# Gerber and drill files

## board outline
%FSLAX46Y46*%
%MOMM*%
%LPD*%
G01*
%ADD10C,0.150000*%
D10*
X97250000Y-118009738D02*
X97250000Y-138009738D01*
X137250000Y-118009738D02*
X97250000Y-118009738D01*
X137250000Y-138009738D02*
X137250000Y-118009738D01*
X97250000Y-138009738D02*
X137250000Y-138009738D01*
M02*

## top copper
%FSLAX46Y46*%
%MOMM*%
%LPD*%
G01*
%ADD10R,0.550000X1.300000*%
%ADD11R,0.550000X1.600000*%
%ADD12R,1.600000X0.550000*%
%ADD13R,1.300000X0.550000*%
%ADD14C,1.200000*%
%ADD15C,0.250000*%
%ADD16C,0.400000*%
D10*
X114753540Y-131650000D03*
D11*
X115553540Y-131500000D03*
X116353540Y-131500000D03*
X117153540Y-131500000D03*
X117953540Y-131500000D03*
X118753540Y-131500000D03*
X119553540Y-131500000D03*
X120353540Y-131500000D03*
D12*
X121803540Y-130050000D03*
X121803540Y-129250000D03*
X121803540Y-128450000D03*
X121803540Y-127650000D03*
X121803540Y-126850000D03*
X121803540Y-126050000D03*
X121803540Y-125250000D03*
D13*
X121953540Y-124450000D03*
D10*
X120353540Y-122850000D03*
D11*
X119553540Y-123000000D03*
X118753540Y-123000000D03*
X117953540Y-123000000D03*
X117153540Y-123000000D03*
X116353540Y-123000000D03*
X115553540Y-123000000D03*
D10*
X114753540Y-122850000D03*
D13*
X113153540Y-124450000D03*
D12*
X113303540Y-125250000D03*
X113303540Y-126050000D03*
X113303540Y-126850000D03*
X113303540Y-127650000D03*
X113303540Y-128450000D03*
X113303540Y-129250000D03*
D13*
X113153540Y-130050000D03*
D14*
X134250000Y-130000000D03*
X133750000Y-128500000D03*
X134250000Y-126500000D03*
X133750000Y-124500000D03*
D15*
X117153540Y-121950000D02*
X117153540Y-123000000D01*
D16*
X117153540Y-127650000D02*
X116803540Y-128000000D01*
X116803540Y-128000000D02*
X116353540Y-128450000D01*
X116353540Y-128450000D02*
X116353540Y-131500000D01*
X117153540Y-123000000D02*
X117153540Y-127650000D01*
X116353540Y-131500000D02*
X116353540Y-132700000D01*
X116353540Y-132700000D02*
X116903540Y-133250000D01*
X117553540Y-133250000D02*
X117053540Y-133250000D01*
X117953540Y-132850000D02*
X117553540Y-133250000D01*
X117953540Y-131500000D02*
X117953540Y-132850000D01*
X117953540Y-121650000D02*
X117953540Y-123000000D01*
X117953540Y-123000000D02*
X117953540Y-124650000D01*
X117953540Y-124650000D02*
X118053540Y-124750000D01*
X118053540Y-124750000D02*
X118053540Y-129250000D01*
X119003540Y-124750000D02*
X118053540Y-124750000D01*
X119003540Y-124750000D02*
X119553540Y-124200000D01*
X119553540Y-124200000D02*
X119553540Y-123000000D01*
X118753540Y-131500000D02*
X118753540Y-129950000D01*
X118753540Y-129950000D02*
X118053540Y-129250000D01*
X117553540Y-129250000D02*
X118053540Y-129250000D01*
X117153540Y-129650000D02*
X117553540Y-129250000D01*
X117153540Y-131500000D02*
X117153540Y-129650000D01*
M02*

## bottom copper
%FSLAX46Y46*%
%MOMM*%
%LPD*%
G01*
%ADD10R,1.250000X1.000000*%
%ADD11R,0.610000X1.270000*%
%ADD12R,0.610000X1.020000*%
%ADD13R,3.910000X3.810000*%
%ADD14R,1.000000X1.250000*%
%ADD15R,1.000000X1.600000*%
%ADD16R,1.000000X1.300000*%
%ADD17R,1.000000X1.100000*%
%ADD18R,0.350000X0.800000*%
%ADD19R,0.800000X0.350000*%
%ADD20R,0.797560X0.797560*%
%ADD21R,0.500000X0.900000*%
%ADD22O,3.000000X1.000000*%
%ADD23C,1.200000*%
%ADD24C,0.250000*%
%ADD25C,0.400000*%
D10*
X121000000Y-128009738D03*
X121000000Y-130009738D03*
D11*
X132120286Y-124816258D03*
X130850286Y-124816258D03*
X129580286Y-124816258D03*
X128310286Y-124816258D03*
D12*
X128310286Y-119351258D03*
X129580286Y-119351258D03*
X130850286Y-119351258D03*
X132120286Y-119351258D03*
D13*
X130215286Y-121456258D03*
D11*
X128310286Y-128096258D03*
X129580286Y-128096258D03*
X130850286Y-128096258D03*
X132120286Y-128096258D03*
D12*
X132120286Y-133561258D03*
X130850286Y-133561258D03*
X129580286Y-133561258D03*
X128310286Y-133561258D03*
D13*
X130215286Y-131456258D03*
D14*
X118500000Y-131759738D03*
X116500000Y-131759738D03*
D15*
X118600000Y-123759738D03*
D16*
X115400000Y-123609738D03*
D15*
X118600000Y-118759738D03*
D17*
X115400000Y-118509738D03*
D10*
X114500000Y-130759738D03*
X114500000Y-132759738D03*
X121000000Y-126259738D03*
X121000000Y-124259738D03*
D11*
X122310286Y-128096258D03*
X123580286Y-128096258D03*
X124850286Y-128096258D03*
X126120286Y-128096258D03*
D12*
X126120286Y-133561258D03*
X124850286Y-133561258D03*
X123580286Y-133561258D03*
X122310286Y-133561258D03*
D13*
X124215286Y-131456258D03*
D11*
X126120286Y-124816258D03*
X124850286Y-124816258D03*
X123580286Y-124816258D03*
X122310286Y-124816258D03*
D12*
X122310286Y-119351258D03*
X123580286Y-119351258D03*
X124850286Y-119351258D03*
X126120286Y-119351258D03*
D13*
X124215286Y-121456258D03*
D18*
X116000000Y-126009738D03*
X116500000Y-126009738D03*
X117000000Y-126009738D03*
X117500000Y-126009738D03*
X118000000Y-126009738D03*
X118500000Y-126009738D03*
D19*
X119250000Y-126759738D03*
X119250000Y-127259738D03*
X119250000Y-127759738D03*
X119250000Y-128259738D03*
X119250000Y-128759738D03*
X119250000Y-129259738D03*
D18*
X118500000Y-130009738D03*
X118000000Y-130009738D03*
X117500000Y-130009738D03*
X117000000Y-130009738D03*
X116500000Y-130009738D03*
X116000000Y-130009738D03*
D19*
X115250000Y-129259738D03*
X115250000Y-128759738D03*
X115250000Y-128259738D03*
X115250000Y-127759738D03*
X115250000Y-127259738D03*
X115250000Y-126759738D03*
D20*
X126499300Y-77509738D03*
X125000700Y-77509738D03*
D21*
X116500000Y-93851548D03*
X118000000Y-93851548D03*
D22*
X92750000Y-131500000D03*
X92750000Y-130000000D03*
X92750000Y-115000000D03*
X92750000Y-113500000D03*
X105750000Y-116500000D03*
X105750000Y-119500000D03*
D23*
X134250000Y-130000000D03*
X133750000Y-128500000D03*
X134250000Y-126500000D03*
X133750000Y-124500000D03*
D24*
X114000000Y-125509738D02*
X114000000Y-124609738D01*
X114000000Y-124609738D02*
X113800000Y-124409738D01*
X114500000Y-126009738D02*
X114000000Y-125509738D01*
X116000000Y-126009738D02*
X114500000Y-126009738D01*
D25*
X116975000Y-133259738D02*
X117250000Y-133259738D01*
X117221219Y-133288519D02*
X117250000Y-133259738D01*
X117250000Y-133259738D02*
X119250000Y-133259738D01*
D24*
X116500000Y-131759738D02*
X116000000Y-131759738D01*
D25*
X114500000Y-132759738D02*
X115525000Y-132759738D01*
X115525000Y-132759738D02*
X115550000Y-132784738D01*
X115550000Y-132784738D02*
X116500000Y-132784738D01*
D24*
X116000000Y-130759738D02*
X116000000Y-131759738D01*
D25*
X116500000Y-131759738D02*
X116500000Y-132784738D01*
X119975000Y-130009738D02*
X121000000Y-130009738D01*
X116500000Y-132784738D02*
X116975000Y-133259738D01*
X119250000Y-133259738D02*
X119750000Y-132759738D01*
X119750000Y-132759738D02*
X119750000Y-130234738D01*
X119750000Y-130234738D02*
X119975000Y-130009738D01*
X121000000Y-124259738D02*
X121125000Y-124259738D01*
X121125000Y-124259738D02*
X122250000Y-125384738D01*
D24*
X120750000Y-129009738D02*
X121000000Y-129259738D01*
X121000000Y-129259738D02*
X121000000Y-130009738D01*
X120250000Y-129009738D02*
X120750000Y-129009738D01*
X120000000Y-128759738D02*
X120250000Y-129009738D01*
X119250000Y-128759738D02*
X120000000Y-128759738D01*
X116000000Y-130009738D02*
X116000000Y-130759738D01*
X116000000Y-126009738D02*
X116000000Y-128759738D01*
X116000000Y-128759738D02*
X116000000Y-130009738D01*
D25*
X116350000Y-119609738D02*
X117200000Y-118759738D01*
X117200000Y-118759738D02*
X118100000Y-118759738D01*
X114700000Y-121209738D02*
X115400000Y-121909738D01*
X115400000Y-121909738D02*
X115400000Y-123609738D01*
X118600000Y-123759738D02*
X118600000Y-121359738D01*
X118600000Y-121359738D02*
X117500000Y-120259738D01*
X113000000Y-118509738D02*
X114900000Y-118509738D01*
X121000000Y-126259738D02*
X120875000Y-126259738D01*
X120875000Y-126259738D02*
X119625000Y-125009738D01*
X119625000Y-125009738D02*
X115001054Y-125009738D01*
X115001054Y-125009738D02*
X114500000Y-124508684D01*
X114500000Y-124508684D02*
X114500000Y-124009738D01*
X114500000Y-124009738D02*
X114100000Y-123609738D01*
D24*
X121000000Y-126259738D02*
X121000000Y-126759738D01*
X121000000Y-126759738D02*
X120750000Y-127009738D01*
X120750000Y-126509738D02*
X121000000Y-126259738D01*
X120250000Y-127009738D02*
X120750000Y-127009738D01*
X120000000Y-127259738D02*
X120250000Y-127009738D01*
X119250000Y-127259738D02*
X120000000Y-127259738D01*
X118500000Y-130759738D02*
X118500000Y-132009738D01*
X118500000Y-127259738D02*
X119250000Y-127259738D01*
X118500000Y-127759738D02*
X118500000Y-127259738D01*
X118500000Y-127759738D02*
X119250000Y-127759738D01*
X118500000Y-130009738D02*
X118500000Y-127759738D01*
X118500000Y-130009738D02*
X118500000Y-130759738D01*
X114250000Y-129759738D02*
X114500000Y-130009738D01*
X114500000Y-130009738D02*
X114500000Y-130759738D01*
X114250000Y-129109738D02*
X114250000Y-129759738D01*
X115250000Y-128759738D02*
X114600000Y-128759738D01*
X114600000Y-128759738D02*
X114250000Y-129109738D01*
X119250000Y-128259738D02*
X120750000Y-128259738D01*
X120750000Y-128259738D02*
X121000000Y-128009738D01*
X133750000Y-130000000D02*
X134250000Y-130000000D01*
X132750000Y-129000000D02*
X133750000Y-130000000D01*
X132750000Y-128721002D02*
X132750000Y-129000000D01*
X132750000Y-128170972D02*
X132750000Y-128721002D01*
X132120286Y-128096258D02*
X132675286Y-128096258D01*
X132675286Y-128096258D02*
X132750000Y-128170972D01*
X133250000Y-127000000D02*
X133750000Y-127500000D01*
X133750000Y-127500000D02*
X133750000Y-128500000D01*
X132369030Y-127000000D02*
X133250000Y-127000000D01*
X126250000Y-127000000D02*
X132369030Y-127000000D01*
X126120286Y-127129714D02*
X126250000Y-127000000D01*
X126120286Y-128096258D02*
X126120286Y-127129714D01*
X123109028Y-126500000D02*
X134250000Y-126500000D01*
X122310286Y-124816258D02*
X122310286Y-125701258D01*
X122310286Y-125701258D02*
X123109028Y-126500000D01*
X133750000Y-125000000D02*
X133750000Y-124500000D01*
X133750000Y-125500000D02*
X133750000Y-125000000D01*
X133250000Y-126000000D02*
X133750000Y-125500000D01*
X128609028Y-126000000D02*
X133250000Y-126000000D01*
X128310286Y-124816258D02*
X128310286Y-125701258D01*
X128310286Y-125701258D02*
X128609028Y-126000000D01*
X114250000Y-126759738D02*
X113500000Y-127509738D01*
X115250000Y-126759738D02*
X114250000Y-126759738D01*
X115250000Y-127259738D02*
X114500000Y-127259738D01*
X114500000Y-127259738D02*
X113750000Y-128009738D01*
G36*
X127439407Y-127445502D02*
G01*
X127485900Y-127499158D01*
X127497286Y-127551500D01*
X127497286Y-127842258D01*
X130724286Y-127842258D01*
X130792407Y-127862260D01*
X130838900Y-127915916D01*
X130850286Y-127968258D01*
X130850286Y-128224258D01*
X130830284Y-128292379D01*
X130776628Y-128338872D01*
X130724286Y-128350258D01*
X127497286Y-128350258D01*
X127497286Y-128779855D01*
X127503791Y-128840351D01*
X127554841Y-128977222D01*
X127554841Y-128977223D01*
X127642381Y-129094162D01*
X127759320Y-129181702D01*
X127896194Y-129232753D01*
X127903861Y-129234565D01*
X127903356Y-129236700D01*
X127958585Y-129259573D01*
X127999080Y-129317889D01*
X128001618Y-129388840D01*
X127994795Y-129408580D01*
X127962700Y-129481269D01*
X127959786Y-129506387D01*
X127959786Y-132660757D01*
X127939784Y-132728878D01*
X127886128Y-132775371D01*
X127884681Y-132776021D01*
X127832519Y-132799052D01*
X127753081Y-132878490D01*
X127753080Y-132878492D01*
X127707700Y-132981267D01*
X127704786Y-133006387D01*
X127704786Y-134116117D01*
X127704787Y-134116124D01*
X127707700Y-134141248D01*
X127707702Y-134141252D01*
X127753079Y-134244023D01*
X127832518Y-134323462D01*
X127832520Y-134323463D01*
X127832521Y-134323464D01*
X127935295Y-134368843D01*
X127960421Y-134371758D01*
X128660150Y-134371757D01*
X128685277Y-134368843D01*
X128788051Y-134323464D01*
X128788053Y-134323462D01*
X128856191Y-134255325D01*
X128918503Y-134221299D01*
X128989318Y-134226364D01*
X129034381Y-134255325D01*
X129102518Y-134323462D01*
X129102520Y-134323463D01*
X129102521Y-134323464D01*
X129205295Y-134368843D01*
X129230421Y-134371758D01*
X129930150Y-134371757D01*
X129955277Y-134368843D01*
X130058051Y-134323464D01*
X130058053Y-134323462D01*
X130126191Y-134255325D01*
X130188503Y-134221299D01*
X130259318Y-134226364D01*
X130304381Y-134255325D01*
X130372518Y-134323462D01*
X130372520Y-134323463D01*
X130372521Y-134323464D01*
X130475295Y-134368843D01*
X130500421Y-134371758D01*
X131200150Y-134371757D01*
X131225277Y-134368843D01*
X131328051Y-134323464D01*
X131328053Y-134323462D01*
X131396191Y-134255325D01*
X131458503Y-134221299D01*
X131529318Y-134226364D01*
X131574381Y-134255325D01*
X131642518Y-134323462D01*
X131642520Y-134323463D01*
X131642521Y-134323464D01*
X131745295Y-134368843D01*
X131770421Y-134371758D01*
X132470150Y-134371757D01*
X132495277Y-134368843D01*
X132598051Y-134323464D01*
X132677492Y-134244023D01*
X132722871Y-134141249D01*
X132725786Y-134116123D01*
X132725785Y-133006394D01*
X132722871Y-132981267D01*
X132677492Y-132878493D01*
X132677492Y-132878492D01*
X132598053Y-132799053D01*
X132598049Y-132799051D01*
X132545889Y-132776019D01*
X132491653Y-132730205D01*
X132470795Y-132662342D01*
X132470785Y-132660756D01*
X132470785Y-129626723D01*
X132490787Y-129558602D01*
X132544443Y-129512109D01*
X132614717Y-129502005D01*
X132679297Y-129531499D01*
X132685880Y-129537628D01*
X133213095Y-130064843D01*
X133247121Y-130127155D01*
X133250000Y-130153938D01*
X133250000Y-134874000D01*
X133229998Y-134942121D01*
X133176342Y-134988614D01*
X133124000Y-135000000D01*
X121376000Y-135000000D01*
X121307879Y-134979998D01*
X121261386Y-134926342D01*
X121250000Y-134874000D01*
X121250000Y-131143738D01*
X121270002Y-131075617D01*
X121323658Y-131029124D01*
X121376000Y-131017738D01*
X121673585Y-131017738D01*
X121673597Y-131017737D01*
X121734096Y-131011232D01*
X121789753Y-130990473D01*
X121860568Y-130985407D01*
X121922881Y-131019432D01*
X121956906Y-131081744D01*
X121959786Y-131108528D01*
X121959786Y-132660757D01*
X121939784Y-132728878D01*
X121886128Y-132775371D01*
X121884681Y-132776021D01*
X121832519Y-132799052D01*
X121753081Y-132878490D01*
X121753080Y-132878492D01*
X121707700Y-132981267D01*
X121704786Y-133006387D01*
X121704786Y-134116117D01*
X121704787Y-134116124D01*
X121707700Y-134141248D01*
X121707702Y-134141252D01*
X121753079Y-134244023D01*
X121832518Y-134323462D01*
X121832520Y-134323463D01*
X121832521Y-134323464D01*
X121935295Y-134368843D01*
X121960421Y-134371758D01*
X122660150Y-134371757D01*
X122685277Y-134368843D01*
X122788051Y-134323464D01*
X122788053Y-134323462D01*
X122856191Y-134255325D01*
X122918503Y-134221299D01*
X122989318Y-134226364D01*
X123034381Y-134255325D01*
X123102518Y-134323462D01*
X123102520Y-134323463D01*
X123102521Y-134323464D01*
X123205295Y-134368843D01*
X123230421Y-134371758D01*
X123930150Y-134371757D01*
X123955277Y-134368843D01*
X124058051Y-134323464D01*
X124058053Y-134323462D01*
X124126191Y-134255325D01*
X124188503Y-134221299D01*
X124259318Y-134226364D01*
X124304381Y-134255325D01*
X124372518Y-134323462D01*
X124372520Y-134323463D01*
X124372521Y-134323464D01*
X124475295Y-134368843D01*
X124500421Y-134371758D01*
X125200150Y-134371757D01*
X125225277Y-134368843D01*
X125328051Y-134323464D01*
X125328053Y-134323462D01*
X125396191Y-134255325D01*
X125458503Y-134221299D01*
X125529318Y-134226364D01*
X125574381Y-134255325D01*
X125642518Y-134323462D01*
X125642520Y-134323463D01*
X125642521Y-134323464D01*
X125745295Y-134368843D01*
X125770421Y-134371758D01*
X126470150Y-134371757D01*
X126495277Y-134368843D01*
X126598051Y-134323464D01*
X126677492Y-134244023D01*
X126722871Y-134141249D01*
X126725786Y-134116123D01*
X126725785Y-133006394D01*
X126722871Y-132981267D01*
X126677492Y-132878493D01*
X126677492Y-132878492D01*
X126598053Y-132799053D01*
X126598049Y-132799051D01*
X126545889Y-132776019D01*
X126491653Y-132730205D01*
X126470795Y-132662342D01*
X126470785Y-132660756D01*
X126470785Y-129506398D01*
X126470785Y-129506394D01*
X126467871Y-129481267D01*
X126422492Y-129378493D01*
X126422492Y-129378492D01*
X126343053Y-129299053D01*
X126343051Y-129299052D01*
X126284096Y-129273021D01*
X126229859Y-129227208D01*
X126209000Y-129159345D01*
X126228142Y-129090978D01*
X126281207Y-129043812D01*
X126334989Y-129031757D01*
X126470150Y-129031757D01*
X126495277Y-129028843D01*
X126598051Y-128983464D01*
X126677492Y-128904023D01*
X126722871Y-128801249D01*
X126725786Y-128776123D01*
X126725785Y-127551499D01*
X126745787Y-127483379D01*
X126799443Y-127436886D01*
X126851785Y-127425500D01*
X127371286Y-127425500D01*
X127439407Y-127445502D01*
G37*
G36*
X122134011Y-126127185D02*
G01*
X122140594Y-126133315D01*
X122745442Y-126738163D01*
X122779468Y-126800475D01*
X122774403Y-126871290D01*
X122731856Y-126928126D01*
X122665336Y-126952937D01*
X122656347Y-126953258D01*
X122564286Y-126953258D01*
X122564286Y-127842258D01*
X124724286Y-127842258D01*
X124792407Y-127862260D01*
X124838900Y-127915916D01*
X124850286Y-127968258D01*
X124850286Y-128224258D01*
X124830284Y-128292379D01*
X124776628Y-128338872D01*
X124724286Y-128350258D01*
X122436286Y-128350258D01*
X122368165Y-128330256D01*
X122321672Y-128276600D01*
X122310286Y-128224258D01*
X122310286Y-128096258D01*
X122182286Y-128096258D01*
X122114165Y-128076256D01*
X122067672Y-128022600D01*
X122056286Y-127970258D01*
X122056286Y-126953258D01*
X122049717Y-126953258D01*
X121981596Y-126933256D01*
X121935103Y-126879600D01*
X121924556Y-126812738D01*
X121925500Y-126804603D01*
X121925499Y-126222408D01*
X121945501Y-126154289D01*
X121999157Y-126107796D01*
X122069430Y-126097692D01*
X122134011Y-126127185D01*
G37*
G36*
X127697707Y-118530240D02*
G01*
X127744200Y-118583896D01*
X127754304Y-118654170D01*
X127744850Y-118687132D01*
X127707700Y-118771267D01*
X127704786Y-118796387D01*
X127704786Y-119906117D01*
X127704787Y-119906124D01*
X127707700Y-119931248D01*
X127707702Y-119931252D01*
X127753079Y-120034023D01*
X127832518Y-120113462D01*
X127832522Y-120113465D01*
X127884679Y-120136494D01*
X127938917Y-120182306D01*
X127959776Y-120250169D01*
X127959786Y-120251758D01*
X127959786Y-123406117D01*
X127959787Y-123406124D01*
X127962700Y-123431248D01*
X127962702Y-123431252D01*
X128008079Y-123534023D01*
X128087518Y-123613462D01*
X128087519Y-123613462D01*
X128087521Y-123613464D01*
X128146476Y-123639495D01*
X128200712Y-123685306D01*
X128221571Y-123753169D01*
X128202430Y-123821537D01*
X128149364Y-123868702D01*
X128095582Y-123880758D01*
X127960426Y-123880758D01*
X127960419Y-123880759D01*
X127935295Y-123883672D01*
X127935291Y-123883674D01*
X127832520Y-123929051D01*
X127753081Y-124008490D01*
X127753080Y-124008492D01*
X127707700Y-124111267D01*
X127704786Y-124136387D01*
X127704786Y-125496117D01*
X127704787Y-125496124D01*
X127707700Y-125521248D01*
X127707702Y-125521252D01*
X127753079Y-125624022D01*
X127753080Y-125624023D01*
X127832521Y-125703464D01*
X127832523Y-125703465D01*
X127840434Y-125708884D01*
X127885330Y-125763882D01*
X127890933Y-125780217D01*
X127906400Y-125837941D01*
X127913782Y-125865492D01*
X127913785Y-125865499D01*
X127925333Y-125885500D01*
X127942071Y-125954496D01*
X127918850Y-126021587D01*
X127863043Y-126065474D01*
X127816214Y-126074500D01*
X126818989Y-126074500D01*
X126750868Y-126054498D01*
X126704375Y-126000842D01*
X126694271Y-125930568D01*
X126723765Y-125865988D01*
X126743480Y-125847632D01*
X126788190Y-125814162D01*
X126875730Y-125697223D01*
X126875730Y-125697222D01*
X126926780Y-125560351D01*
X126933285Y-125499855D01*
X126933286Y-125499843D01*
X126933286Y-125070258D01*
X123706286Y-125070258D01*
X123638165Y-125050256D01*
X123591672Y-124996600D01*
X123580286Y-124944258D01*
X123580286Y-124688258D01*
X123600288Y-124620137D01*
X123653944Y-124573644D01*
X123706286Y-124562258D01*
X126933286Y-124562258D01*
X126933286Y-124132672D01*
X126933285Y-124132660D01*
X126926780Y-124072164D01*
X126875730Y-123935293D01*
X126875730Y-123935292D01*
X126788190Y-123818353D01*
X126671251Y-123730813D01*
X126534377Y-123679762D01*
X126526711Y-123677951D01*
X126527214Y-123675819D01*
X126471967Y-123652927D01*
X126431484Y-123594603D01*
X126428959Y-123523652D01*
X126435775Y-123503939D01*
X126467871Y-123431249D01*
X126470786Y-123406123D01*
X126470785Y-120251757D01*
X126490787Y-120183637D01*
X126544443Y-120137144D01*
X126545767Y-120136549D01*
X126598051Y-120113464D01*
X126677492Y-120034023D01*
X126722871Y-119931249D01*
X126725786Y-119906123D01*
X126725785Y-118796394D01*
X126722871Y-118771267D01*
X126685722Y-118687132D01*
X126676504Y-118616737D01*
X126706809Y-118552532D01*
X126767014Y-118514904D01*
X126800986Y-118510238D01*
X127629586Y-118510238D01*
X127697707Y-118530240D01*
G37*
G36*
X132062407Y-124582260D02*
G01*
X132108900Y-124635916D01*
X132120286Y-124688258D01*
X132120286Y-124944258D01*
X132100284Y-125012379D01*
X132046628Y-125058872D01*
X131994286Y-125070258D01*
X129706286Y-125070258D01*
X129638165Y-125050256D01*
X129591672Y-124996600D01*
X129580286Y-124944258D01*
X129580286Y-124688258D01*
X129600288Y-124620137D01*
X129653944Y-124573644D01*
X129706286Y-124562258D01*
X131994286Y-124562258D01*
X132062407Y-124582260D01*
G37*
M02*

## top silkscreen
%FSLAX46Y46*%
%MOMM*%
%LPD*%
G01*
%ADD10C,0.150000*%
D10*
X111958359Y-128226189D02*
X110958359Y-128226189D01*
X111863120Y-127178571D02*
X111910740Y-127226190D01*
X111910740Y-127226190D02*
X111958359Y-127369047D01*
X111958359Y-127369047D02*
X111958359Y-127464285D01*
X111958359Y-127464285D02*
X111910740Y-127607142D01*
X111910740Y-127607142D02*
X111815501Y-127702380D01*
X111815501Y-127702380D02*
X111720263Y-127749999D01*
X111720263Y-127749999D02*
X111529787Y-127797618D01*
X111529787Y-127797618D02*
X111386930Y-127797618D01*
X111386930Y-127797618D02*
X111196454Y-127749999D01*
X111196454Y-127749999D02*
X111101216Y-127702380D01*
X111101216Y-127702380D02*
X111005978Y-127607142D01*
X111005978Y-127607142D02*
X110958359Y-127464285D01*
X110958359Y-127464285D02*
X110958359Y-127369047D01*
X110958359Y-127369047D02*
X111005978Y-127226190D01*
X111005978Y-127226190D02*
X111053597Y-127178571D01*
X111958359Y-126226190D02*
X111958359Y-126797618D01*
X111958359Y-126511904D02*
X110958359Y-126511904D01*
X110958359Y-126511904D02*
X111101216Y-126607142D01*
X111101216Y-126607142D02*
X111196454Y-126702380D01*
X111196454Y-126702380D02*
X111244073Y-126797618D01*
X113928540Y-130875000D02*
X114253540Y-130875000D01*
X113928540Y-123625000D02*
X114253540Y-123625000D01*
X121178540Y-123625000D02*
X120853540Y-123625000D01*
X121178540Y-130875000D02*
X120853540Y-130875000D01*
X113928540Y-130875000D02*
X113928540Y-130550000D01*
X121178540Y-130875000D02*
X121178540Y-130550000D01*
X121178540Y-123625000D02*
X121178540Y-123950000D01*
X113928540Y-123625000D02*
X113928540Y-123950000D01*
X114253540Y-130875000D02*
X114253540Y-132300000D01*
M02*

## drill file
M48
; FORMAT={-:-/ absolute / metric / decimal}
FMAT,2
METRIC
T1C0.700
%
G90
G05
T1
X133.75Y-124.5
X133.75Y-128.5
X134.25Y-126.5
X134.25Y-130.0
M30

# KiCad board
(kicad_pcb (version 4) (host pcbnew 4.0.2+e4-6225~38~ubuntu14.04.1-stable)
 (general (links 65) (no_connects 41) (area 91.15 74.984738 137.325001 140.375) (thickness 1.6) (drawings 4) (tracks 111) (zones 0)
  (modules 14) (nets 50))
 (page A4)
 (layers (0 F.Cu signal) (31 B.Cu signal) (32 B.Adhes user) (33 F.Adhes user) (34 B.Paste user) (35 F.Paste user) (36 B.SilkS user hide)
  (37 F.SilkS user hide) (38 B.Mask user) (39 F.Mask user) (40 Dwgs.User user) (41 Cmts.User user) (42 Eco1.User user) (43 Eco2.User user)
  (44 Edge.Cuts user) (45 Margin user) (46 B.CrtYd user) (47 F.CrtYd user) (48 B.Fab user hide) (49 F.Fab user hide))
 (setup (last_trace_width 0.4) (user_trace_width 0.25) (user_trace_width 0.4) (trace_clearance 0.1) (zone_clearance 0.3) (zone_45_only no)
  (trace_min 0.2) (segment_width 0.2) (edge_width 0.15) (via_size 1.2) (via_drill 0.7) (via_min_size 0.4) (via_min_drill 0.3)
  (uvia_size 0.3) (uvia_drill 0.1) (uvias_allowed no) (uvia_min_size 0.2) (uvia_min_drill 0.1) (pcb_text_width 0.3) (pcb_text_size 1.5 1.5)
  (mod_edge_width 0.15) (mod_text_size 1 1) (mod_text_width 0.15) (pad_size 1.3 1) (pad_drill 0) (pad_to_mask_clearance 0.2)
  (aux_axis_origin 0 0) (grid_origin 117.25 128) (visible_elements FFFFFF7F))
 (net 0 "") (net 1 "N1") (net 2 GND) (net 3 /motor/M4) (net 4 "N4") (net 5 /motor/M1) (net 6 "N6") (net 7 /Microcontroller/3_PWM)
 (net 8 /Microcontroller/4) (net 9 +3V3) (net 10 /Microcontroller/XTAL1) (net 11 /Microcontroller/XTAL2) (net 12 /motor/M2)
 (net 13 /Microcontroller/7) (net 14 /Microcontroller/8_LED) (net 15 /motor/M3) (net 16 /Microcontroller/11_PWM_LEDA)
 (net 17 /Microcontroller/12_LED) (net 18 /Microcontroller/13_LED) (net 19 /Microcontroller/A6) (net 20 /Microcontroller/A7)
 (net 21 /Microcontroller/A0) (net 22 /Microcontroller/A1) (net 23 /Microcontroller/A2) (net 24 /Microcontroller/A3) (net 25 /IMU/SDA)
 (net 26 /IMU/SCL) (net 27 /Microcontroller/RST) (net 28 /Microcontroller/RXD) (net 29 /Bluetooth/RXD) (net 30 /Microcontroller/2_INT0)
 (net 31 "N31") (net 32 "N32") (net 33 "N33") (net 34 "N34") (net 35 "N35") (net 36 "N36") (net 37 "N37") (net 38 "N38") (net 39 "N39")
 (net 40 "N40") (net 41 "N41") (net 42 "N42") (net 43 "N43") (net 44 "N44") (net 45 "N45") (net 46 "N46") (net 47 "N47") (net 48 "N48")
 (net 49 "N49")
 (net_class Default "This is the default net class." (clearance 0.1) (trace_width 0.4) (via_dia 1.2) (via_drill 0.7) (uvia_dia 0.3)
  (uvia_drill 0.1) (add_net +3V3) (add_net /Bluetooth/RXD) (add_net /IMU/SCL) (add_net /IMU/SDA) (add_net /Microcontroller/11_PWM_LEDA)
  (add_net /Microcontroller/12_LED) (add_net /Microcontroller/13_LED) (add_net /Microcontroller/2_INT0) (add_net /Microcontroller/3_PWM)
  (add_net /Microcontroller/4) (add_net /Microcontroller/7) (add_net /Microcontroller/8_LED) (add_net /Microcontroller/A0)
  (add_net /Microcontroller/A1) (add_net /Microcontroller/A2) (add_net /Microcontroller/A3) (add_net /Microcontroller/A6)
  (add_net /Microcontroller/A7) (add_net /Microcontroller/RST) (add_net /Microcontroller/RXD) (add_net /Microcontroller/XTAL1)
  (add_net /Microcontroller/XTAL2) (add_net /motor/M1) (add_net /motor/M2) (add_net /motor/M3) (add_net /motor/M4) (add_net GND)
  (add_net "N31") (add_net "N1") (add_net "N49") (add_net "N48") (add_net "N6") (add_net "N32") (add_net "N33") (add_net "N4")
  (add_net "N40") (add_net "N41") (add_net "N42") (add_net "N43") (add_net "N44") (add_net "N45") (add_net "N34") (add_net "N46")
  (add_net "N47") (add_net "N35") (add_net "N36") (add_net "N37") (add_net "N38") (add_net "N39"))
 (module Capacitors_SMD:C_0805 (layer B.Cu) (at 121 129.009738 270)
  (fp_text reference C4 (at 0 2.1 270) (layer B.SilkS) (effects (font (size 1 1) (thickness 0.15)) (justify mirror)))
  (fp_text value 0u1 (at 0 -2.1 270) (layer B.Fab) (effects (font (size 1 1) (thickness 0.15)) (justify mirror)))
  (pad 1 smd rect (at -1 0 270) (size 1 1.25) (layers B.Cu B.Paste B.Mask) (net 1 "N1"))
  (pad 2 smd rect (at 1 0 270) (size 1 1.25) (layers B.Cu B.Paste B.Mask) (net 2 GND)))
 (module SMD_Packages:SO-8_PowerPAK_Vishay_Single (layer B.Cu) (at 130.215286 122.146258 90)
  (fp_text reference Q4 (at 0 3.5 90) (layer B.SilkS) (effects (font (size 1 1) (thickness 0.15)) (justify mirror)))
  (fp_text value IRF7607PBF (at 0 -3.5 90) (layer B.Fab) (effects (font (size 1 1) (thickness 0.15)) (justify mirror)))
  (pad 1 smd rect (at -2.67 1.905 90) (size 1.27 0.61) (layers B.Cu B.Paste B.Mask) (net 2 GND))
  (pad 2 smd rect (at -2.67 0.635 90) (size 1.27 0.61) (layers B.Cu B.Paste B.Mask) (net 2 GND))
  (pad 3 smd rect (at -2.67 -0.635 90) (size 1.27 0.61) (layers B.Cu B.Paste B.Mask) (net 2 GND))
  (pad 4 smd rect (at -2.67 -1.905 90) (size 1.27 0.61) (layers B.Cu B.Paste B.Mask) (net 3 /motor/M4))
  (pad 5 smd rect (at 2.795 -1.905 90) (size 1.02 0.61) (layers B.Cu B.Paste B.Mask) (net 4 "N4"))
  (pad 5 smd rect (at 2.795 -0.635 90) (size 1.02 0.61) (layers B.Cu B.Paste B.Mask) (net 4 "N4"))
  (pad 5 smd rect (at 2.795 0.635 90) (size 1.02 0.61) (layers B.Cu B.Paste B.Mask) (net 4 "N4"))
  (pad 5 smd rect (at 2.795 1.905 90) (size 1.02 0.61) (layers B.Cu B.Paste B.Mask) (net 4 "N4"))
  (pad 5 smd rect (at 0.69 0 90) (size 3.81 3.91) (layers B.Cu B.Paste B.Mask) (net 4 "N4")))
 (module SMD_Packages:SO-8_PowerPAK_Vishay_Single (layer B.Cu) (at 130.215286 130.766258 270)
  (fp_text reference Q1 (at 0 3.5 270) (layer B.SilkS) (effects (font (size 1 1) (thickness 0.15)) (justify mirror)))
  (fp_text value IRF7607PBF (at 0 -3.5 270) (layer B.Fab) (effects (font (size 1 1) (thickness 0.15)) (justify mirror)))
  (pad 1 smd rect (at -2.67 1.905 270) (size 1.27 0.61) (layers B.Cu B.Paste B.Mask) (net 2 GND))
  (pad 2 smd rect (at -2.67 0.635 270) (size 1.27 0.61) (layers B.Cu B.Paste B.Mask) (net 2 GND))
  (pad 3 smd rect (at -2.67 -0.635 270) (size 1.27 0.61) (layers B.Cu B.Paste B.Mask) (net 2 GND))
  (pad 4 smd rect (at -2.67 -1.905 270) (size 1.27 0.61) (layers B.Cu B.Paste B.Mask) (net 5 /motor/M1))
  (pad 5 smd rect (at 2.795 -1.905 270) (size 1.02 0.61) (layers B.Cu B.Paste B.Mask) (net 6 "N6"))
  (pad 5 smd rect (at 2.795 -0.635 270) (size 1.02 0.61) (layers B.Cu B.Paste B.Mask) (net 6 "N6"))
  (pad 5 smd rect (at 2.795 0.635 270) (size 1.02 0.61) (layers B.Cu B.Paste B.Mask) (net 6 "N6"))
  (pad 5 smd rect (at 2.795 1.905 270) (size 1.02 0.61) (layers B.Cu B.Paste B.Mask) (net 6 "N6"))
  (pad 5 smd rect (at 0.69 0 270) (size 3.81 3.91) (layers B.Cu B.Paste B.Mask) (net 6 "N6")))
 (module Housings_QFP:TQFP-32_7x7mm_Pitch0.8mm (layer F.Cu) (at 117.55354 127.25 90)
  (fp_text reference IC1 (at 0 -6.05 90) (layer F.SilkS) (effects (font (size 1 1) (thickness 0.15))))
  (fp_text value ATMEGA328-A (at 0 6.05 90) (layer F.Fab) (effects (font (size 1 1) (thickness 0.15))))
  (fp_line (start -3.625 -3.625) (end -3.625 -3.3) (layer F.SilkS) (width 0.15))
  (fp_line (start 3.625 -3.625) (end 3.625 -3.3) (layer F.SilkS) (width 0.15))
  (fp_line (start 3.625 3.625) (end 3.625 3.3) (layer F.SilkS) (width 0.15))
  (fp_line (start -3.625 3.625) (end -3.625 3.3) (layer F.SilkS) (width 0.15))
  (fp_line (start -3.625 -3.625) (end -3.3 -3.625) (layer F.SilkS) (width 0.15))
  (fp_line (start -3.625 3.625) (end -3.3 3.625) (layer F.SilkS) (width 0.15))
  (fp_line (start 3.625 3.625) (end 3.3 3.625) (layer F.SilkS) (width 0.15))
  (fp_line (start 3.625 -3.625) (end 3.3 -3.625) (layer F.SilkS) (width 0.15))
  (fp_line (start -3.625 -3.3) (end -5.05 -3.3) (layer F.SilkS) (width 0.15))
  (pad 1 smd rect (at -4.4 -2.8 90) (size 1.3 0.55) (layers F.Cu F.Paste F.Mask) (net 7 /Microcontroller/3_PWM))
  (pad 2 smd rect (at -4.25 -2 90) (size 1.6 0.55) (layers F.Cu F.Paste F.Mask) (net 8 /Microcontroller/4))
  (pad 3 smd rect (at -4.25 -1.2 90) (size 1.6 0.55) (layers F.Cu F.Paste F.Mask) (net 2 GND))
  (pad 4 smd rect (at -4.25 -0.4 90) (size 1.6 0.55) (layers F.Cu F.Paste F.Mask) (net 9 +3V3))
  (pad 5 smd rect (at -4.25 0.4 90) (size 1.6 0.55) (layers F.Cu F.Paste F.Mask) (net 2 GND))
  (pad 6 smd rect (at -4.25 1.2 90) (size 1.6 0.55) (layers F.Cu F.Paste F.Mask) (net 9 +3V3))
  (pad 7 smd rect (at -4.25 2 90) (size 1.6 0.55) (layers F.Cu F.Paste F.Mask) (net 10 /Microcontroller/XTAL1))
  (pad 8 smd rect (at -4.25 2.8 90) (size 1.6 0.55) (layers F.Cu F.Paste F.Mask) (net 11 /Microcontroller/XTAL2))
  (pad 9 smd rect (at -2.8 4.25 180) (size 1.6 0.55) (layers F.Cu F.Paste F.Mask) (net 5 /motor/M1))
  (pad 10 smd rect (at -2 4.25 180) (size 1.6 0.55) (layers F.Cu F.Paste F.Mask) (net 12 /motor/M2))
  (pad 11 smd rect (at -1.2 4.25 180) (size 1.6 0.55) (layers F.Cu F.Paste F.Mask) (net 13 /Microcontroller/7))
  (pad 12 smd rect (at -0.4 4.25 180) (size 1.6 0.55) (layers F.Cu F.Paste F.Mask) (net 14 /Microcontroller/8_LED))
  (pad 13 smd rect (at 0.4 4.25 180) (size 1.6 0.55) (layers F.Cu F.Paste F.Mask) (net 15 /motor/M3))
  (pad 14 smd rect (at 1.2 4.25 180) (size 1.6 0.55) (layers F.Cu F.Paste F.Mask) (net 3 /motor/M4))
  (pad 15 smd rect (at 2 4.25 180) (size 1.6 0.55) (layers F.Cu F.Paste F.Mask) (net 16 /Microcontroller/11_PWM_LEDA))
  (pad 16 smd rect (at 2.8 4.4 180) (size 1.3 0.55) (layers F.Cu F.Paste F.Mask) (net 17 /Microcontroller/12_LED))
  (pad 17 smd rect (at 4.4 2.8 90) (size 1.3 0.55) (layers F.Cu F.Paste F.Mask) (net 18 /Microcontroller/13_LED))
  (pad 18 smd rect (at 4.25 2 90) (size 1.6 0.55) (layers F.Cu F.Paste F.Mask) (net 9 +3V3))
  (pad 19 smd rect (at 4.25 1.2 90) (size 1.6 0.55) (layers F.Cu F.Paste F.Mask) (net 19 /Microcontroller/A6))
  (pad 20 smd rect (at 4.25 0.4 90) (size 1.6 0.55) (layers F.Cu F.Paste F.Mask) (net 9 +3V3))
  (pad 21 smd rect (at 4.25 -0.4 90) (size 1.6 0.55) (layers F.Cu F.Paste F.Mask) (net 2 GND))
  (pad 22 smd rect (at 4.25 -1.2 90) (size 1.6 0.55) (layers F.Cu F.Paste F.Mask) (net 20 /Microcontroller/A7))
  (pad 23 smd rect (at 4.25 -2 90) (size 1.6 0.55) (layers F.Cu F.Paste F.Mask) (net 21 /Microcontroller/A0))
  (pad 24 smd rect (at 4.4 -2.8 90) (size 1.3 0.55) (layers F.Cu F.Paste F.Mask) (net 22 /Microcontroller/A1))
  (pad 25 smd rect (at 2.8 -4.4 180) (size 1.3 0.55) (layers F.Cu F.Paste F.Mask) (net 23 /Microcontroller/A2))
  (pad 26 smd rect (at 2 -4.25 180) (size 1.6 0.55) (layers F.Cu F.Paste F.Mask) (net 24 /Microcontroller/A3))
  (pad 27 smd rect (at 1.2 -4.25 180) (size 1.6 0.55) (layers F.Cu F.Paste F.Mask) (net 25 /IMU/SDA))
  (pad 28 smd rect (at 0.4 -4.25 180) (size 1.6 0.55) (layers F.Cu F.Paste F.Mask) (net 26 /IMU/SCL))
  (pad 29 smd rect (at -0.4 -4.25 180) (size 1.6 0.55) (layers F.Cu F.Paste F.Mask) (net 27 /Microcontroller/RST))
  (pad 30 smd rect (at -1.2 -4.25 180) (size 1.6 0.55) (layers F.Cu F.Paste F.Mask) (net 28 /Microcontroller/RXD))
  (pad 31 smd rect (at -2 -4.25 180) (size 1.6 0.55) (layers F.Cu F.Paste F.Mask) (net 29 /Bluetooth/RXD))
  (pad 32 smd rect (at -2.8 -4.4 180) (size 1.3 0.55) (layers F.Cu F.Paste F.Mask) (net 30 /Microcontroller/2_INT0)))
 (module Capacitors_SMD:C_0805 (layer B.Cu) (at 117.5 131.759738 180)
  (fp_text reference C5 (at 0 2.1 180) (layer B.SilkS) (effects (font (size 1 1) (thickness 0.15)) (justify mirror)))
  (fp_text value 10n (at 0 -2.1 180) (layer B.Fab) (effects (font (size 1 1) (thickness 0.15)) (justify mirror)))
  (pad 1 smd rect (at -1 0 180) (size 1 1.25) (layers B.Cu B.Paste B.Mask) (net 9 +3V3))
  (pad 2 smd rect (at 1 0 180) (size 1 1.25) (layers B.Cu B.Paste B.Mask) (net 2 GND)))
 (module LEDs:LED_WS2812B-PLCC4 (layer B.Cu) (at 117 121.259738 270)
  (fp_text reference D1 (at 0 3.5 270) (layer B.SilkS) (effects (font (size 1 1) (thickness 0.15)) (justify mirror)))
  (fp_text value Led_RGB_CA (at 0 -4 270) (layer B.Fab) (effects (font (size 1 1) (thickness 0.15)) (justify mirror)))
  (pad 3 smd rect (at 2.5 -1.6 270) (size 1.6 1) (layers B.Cu B.Paste B.Mask) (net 14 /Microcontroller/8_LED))
  (pad 4 smd rect (at 2.35 1.6 270) (size 1.3 1) (layers B.Cu B.Paste B.Mask) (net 18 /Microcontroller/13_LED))
  (pad 2 smd rect (at -2.5 -1.6 270) (size 1.6 1) (layers B.Cu B.Paste B.Mask) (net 17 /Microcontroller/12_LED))
  (pad 1 smd rect (at -2.75 1.6 270) (size 1.1 1) (layers B.Cu B.Paste B.Mask) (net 16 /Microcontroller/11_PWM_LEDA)))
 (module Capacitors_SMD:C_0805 (layer B.Cu) (at 114.5 131.759738 270)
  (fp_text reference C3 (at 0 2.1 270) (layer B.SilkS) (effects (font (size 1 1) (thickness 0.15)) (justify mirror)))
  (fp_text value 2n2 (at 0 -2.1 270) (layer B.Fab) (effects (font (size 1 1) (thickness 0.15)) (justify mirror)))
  (pad 1 smd rect (at -1 0 270) (size 1 1.25) (layers B.Cu B.Paste B.Mask) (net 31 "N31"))
  (pad 2 smd rect (at 1 0 270) (size 1 1.25) (layers B.Cu B.Paste B.Mask) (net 2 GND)))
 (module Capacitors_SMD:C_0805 (layer B.Cu) (at 121 125.259738 90)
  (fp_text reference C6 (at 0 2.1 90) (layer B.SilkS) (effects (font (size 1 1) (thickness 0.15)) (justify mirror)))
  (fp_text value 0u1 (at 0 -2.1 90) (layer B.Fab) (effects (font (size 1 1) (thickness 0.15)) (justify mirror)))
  (pad 1 smd rect (at -1 0 90) (size 1 1.25) (layers B.Cu B.Paste B.Mask) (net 9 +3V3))
  (pad 2 smd rect (at 1 0 90) (size 1 1.25) (layers B.Cu B.Paste B.Mask) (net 2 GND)))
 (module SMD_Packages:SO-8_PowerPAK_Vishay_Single (layer B.Cu) (at 124.215286 130.766258 270)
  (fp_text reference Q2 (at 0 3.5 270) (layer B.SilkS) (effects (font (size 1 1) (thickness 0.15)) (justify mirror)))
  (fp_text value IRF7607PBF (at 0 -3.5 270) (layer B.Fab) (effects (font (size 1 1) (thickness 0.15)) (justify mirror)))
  (pad 1 smd rect (at -2.67 1.905 270) (size 1.27 0.61) (layers B.Cu B.Paste B.Mask) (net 2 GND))
  (pad 2 smd rect (at -2.67 0.635 270) (size 1.27 0.61) (layers B.Cu B.Paste B.Mask) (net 2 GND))
  (pad 3 smd rect (at -2.67 -0.635 270) (size 1.27 0.61) (layers B.Cu B.Paste B.Mask) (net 2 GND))
  (pad 4 smd rect (at -2.67 -1.905 270) (size 1.27 0.61) (layers B.Cu B.Paste B.Mask) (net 12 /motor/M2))
  (pad 5 smd rect (at 2.795 -1.905 270) (size 1.02 0.61) (layers B.Cu B.Paste B.Mask) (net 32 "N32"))
  (pad 5 smd rect (at 2.795 -0.635 270) (size 1.02 0.61) (layers B.Cu B.Paste B.Mask) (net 32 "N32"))
  (pad 5 smd rect (at 2.795 0.635 270) (size 1.02 0.61) (layers B.Cu B.Paste B.Mask) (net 32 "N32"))
  (pad 5 smd rect (at 2.795 1.905 270) (size 1.02 0.61) (layers B.Cu B.Paste B.Mask) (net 32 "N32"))
  (pad 5 smd rect (at 0.69 0 270) (size 3.81 3.91) (layers B.Cu B.Paste B.Mask) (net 32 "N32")))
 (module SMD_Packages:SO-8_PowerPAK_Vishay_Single (layer B.Cu) (at 124.215286 122.146258 90)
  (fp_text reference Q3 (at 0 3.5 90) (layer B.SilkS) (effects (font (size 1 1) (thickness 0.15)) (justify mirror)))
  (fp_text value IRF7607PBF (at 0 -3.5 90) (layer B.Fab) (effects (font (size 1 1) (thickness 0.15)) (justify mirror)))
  (pad 1 smd rect (at -2.67 1.905 90) (size 1.27 0.61) (layers B.Cu B.Paste B.Mask) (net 2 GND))
  (pad 2 smd rect (at -2.67 0.635 90) (size 1.27 0.61) (layers B.Cu B.Paste B.Mask) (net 2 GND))
  (pad 3 smd rect (at -2.67 -0.635 90) (size 1.27 0.61) (layers B.Cu B.Paste B.Mask) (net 2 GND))
  (pad 4 smd rect (at -2.67 -1.905 90) (size 1.27 0.61) (layers B.Cu B.Paste B.Mask) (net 15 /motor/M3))
  (pad 5 smd rect (at 2.795 -1.905 90) (size 1.02 0.61) (layers B.Cu B.Paste B.Mask) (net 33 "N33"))
  (pad 5 smd rect (at 2.795 -0.635 90) (size 1.02 0.61) (layers B.Cu B.Paste B.Mask) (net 33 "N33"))
  (pad 5 smd rect (at 2.795 0.635 90) (size 1.02 0.61) (layers B.Cu B.Paste B.Mask) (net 33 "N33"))
  (pad 5 smd rect (at 2.795 1.905 90) (size 1.02 0.61) (layers B.Cu B.Paste B.Mask) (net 33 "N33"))
  (pad 5 smd rect (at 0.69 0 90) (size 3.81 3.91) (layers B.Cu B.Paste B.Mask) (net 33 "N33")))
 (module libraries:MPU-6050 (layer B.Cu) (at 117.25 128.009738 270)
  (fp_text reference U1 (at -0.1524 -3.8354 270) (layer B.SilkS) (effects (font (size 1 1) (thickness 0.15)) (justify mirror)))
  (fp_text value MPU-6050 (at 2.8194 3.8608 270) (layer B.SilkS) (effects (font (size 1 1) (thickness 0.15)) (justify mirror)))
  (pad 1 smd rect (at -2 1.25 270) (size 0.8 0.35) (layers B.Cu B.Paste B.Mask) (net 2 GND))
  (pad 2 smd rect (at -2 0.75 270) (size 0.8 0.35) (layers B.Cu B.Paste B.Mask) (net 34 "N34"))
  (pad 3 smd rect (at -2 0.25 270) (size 0.8 0.35) (layers B.Cu B.Paste B.Mask) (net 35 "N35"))
  (pad 4 smd rect (at -2 -0.25 270) (size 0.8 0.35) (layers B.Cu B.Paste B.Mask) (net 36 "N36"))
  (pad 5 smd rect (at -2 -0.75 270) (size 0.8 0.35) (layers B.Cu B.Paste B.Mask) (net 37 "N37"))
  (pad 6 smd rect (at -2 -1.25 270) (size 0.8 0.35) (layers B.Cu B.Paste B.Mask) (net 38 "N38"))
  (pad 7 smd rect (at -1.25 -2 270) (size 0.35 0.8) (layers B.Cu B.Paste B.Mask) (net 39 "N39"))
  (pad 8 smd rect (at -0.75 -2 270) (size 0.35 0.8) (layers B.Cu B.Paste B.Mask) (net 9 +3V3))
  (pad 9 smd rect (at -0.25 -2 270) (size 0.35 0.8) (layers B.Cu B.Paste B.Mask) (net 9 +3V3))
  (pad 10 smd rect (at 0.25 -2 270) (size 0.35 0.8) (layers B.Cu B.Paste B.Mask) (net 1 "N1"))
  (pad 11 smd rect (at 0.75 -2 270) (size 0.35 0.8) (layers B.Cu B.Paste B.Mask) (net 2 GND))
  (pad 12 smd rect (at 1.25 -2 270) (size 0.35 0.8) (layers B.Cu B.Paste B.Mask) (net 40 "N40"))
  (pad 13 smd rect (at 2 -1.25 270) (size 0.8 0.35) (layers B.Cu B.Paste B.Mask) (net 9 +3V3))
  (pad 14 smd rect (at 2 -0.75 270) (size 0.8 0.35) (layers B.Cu B.Paste B.Mask) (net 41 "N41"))
  (pad 15 smd rect (at 2 -0.25 270) (size 0.8 0.35) (layers B.Cu B.Paste B.Mask) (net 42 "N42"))
  (pad 16 smd rect (at 2 0.25 270) (size 0.8 0.35) (layers B.Cu B.Paste B.Mask) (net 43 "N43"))
  (pad 17 smd rect (at 2 0.75 270) (size 0.8 0.35) (layers B.Cu B.Paste B.Mask) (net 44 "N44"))
  (pad 18 smd rect (at 2 1.25 270) (size 0.8 0.35) (layers B.Cu B.Paste B.Mask) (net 2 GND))
  (pad 19 smd rect (at 1.25 2 270) (size 0.35 0.8) (layers B.Cu B.Paste B.Mask) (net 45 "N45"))
  (pad 20 smd rect (at 0.75 2 270) (size 0.35 0.8) (layers B.Cu B.Paste B.Mask) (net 31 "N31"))
  (pad 21 smd rect (at 0.25 2 270) (size 0.35 0.8) (layers B.Cu B.Paste B.Mask) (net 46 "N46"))
  (pad 22 smd rect (at -0.25 2 270) (size 0.35 0.8) (layers B.Cu B.Paste B.Mask) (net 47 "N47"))
  (pad 23 smd rect (at -0.75 2 270) (size 0.35 0.8) (layers B.Cu B.Paste B.Mask) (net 26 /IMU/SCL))
  (pad 24 smd rect (at -1.25 2 270) (size 0.35 0.8) (layers B.Cu B.Paste B.Mask) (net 25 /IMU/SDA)))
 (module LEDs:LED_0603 (layer B.Cu) (at 125.75 77.509738)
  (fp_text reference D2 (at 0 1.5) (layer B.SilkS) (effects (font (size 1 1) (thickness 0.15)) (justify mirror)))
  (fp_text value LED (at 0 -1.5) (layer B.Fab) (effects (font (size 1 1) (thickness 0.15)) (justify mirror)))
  (pad 2 smd rect (at 0.7493 0 180) (size 0.79756 0.79756) (layers B.Cu B.Paste B.Mask) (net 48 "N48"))
  (pad 1 smd rect (at -0.7493 0 180) (size 0.79756 0.79756) (layers B.Cu B.Paste B.Mask) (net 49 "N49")))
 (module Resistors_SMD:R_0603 (layer B.Cu) (at 117.25 93.851548)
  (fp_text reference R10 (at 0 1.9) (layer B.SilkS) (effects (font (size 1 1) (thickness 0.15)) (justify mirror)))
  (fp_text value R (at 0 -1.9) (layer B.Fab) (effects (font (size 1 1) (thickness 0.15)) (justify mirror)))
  (pad 1 smd rect (at -0.75 0) (size 0.5 0.9) (layers B.Cu B.Paste B.Mask) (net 49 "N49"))
  (pad 2 smd rect (at 0.75 0) (size 0.5 0.9) (layers B.Cu B.Paste B.Mask) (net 2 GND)))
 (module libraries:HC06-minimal (layer B.Cu) (at 98.75 122.5)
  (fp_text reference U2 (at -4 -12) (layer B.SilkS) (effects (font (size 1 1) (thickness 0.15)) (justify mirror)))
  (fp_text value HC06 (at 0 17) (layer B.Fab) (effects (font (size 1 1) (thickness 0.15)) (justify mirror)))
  (pad 1 smd oval (at -6 9) (size 3 1) (layers B.Cu B.Paste B.Mask) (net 28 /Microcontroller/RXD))
  (pad 2 smd oval (at -6 7.5) (size 3 1) (layers B.Cu B.Paste B.Mask) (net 29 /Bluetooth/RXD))
  (pad 12 smd oval (at -6 -7.5) (size 3 1) (layers B.Cu B.Paste B.Mask) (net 9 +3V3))
  (pad 13 smd oval (at -6 -9) (size 3 1) (layers B.Cu B.Paste B.Mask) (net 2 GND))
  (pad 24 smd oval (at 7 -6) (size 3 1) (layers B.Cu B.Paste B.Mask) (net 48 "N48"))
  (pad 26 smd oval (at 7 -3) (size 3 1) (layers B.Cu B.Paste B.Mask) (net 2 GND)))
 (gr_line (start 97.25 118.009738) (end 97.25 138.009738) (layer Edge.Cuts) (width 0.15))
 (gr_line (start 137.25 118.009738) (end 97.25 118.009738) (layer Edge.Cuts) (width 0.15))
 (gr_line (start 137.25 138.009738) (end 137.25 118.009738) (layer Edge.Cuts) (width 0.15))
 (gr_line (start 97.25 138.009738) (end 137.25 138.009738) (layer Edge.Cuts) (width 0.15))
 (segment (start 114 125.509738) (end 114 124.609738) (width 0.25) (layer B.Cu) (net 2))
 (segment (start 114 124.609738) (end 113.8 124.409738) (width 0.25) (layer B.Cu) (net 2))
 (segment (start 114.5 126.009738) (end 114 125.509738) (width 0.25) (layer B.Cu) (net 2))
 (segment (start 116 126.009738) (end 114.5 126.009738) (width 0.25) (layer B.Cu) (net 2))
 (segment (start 117.15354 121.95) (end 117.15354 123) (width 0.25) (layer F.Cu) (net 2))
 (segment (start 116.975 133.259738) (end 117.25 133.259738) (width 0.4) (layer B.Cu) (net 2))
 (segment (start 117.221219 133.288519) (end 117.25 133.259738) (width 0.4) (layer B.Cu) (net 2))
 (segment (start 117.25 133.259738) (end 119.25 133.259738) (width 0.4) (layer B.Cu) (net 2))
 (segment (start 117.15354 127.65) (end 116.80354 128) (width 0.4) (layer F.Cu) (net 2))
 (segment (start 116.80354 128) (end 116.35354 128.45) (width 0.4) (layer F.Cu) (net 2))
 (segment (start 116.35354 128.45) (end 116.35354 131.5) (width 0.4) (layer F.Cu) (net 2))
 (segment (start 117.15354 123) (end 117.15354 127.65) (width 0.4) (layer F.Cu) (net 2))
 (segment (start 116.35354 131.5) (end 116.35354 132.7) (width 0.4) (layer F.Cu) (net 2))
 (segment (start 116.35354 132.7) (end 116.90354 133.25) (width 0.4) (layer F.Cu) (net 2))
 (segment (start 117.55354 133.25) (end 117.05354 133.25) (width 0.4) (layer F.Cu) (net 2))
 (segment (start 117.95354 132.85) (end 117.55354 133.25) (width 0.4) (layer F.Cu) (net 2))
 (segment (start 117.95354 131.5) (end 117.95354 132.85) (width 0.4) (layer F.Cu) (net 2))
 (segment (start 116.5 131.759738) (end 116 131.759738) (width 0.25) (layer B.Cu) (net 2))
 (segment (start 114.5 132.759738) (end 115.525 132.759738) (width 0.4) (layer B.Cu) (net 2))
 (segment (start 115.525 132.759738) (end 115.55 132.784738) (width 0.4) (layer B.Cu) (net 2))
 (segment (start 115.55 132.784738) (end 116.5 132.784738) (width 0.4) (layer B.Cu) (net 2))
 (segment (start 116 130.759738) (end 116 131.759738) (width 0.25) (layer B.Cu) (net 2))
 (segment (start 116.5 131.759738) (end 116.5 132.784738) (width 0.4) (layer B.Cu) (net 2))
 (segment (start 119.975 130.009738) (end 121 130.009738) (width 0.4) (layer B.Cu) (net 2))
 (segment (start 116.5 132.784738) (end 116.975 133.259738) (width 0.4) (layer B.Cu) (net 2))
 (segment (start 119.25 133.259738) (end 119.75 132.759738) (width 0.4) (layer B.Cu) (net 2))
 (segment (start 119.75 132.759738) (end 119.75 130.234738) (width 0.4) (layer B.Cu) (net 2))
 (segment (start 119.75 130.234738) (end 119.975 130.009738) (width 0.4) (layer B.Cu) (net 2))
 (segment (start 121 124.259738) (end 121.125 124.259738) (width 0.4) (layer B.Cu) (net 2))
 (segment (start 121.125 124.259738) (end 122.25 125.384738) (width 0.4) (layer B.Cu) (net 2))
 (segment (start 120.75 129.009738) (end 121 129.259738) (width 0.25) (layer B.Cu) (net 2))
 (segment (start 121 129.259738) (end 121 130.009738) (width 0.25) (layer B.Cu) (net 2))
 (segment (start 120.25 129.009738) (end 120.75 129.009738) (width 0.25) (layer B.Cu) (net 2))
 (segment (start 120 128.759738) (end 120.25 129.009738) (width 0.25) (layer B.Cu) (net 2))
 (segment (start 119.25 128.759738) (end 120 128.759738) (width 0.25) (layer B.Cu) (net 2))
 (segment (start 116 130.009738) (end 116 130.759738) (width 0.25) (layer B.Cu) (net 2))
 (segment (start 116 126.009738) (end 116 128.759738) (width 0.25) (layer B.Cu) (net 2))
 (segment (start 116 128.759738) (end 116 130.009738) (width 0.25) (layer B.Cu) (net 2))
 (segment (start 116.35 119.609738) (end 117.2 118.759738) (width 0.4) (layer B.Cu) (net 17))
 (segment (start 117.2 118.759738) (end 118.1 118.759738) (width 0.4) (layer B.Cu) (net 17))
 (segment (start 114.7 121.209738) (end 115.4 121.909738) (width 0.4) (layer B.Cu) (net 18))
 (segment (start 115.4 121.909738) (end 115.4 123.609738) (width 0.4) (layer B.Cu) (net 18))
 (segment (start 118.6 123.759738) (end 118.6 121.359738) (width 0.4) (layer B.Cu) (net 14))
 (segment (start 118.6 121.359738) (end 117.5 120.259738) (width 0.4) (layer B.Cu) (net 14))
 (segment (start 113 118.509738) (end 114.9 118.509738) (width 0.4) (layer B.Cu) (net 16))
 (segment (start 121 126.259738) (end 120.875 126.259738) (width 0.4) (layer B.Cu) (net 9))
 (segment (start 120.875 126.259738) (end 119.625 125.009738) (width 0.4) (layer B.Cu) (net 9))
 (segment (start 119.625 125.009738) (end 115.001054 125.009738) (width 0.4) (layer B.Cu) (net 9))
 (segment (start 117.95354 121.65) (end 117.95354 123) (width 0.4) (layer F.Cu) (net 9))
 (segment (start 115.001054 125.009738) (end 114.5 124.508684) (width 0.4) (layer B.Cu) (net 9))
 (segment (start 114.5 124.508684) (end 114.5 124.009738) (width 0.4) (layer B.Cu) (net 9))
 (segment (start 114.5 124.009738) (end 114.1 123.609738) (width 0.4) (layer B.Cu) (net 9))
 (segment (start 117.95354 123) (end 117.95354 124.65) (width 0.4) (layer F.Cu) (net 9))
 (segment (start 117.95354 124.65) (end 118.05354 124.75) (width 0.4) (layer F.Cu) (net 9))
 (segment (start 118.05354 124.75) (end 118.05354 129.25) (width 0.4) (layer F.Cu) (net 9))
 (segment (start 119.00354 124.75) (end 118.05354 124.75) (width 0.4) (layer F.Cu) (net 9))
 (segment (start 119.00354 124.75) (end 119.55354 124.2) (width 0.4) (layer F.Cu) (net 9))
 (segment (start 119.55354 124.2) (end 119.55354 123) (width 0.4) (layer F.Cu) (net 9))
 (segment (start 118.75354 131.5) (end 118.75354 129.95) (width 0.4) (layer F.Cu) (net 9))
 (segment (start 118.75354 129.95) (end 118.05354 129.25) (width 0.4) (layer F.Cu) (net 9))
 (segment (start 117.55354 129.25) (end 118.05354 129.25) (width 0.4) (layer F.Cu) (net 9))
 (segment (start 117.15354 129.65) (end 117.55354 129.25) (width 0.4) (layer F.Cu) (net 9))
 (segment (start 117.15354 131.5) (end 117.15354 129.65) (width 0.4) (layer F.Cu) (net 9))
 (segment (start 121 126.259738) (end 121 126.759738) (width 0.25) (layer B.Cu) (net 9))
 (segment (start 121 126.759738) (end 120.75 127.009738) (width 0.25) (layer B.Cu) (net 9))
 (segment (start 120.75 126.509738) (end 121 126.259738) (width 0.25) (layer B.Cu) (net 9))
 (segment (start 120.25 127.009738) (end 120.75 127.009738) (width 0.25) (layer B.Cu) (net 9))
 (segment (start 120 127.259738) (end 120.25 127.009738) (width 0.25) (layer B.Cu) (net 9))
 (segment (start 119.25 127.259738) (end 120 127.259738) (width 0.25) (layer B.Cu) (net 9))
 (segment (start 118.5 130.759738) (end 118.5 132.009738) (width 0.25) (layer B.Cu) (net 9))
 (segment (start 118.5 127.259738) (end 119.25 127.259738) (width 0.25) (layer B.Cu) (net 9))
 (segment (start 118.5 127.759738) (end 118.5 127.259738) (width 0.25) (layer B.Cu) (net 9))
 (segment (start 118.5 127.759738) (end 119.25 127.759738) (width 0.25) (layer B.Cu) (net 9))
 (segment (start 118.5 130.009738) (end 118.5 127.759738) (width 0.25) (layer B.Cu) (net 9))
 (segment (start 118.5 130.009738) (end 118.5 130.759738) (width 0.25) (layer B.Cu) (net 9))
 (segment (start 114.25 129.759738) (end 114.5 130.009738) (width 0.25) (layer B.Cu) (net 31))
 (segment (start 114.5 130.009738) (end 114.5 130.759738) (width 0.25) (layer B.Cu) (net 31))
 (segment (start 114.25 129.109738) (end 114.25 129.759738) (width 0.25) (layer B.Cu) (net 31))
 (segment (start 115.25 128.759738) (end 114.6 128.759738) (width 0.25) (layer B.Cu) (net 31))
 (segment (start 114.6 128.759738) (end 114.25 129.109738) (width 0.25) (layer B.Cu) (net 31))
 (segment (start 119.25 128.259738) (end 120.75 128.259738) (width 0.25) (layer B.Cu) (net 1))
 (segment (start 120.75 128.259738) (end 121 128.009738) (width 0.25) (layer B.Cu) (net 1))
 (via (at 134.25 130) (size 1.2) (drill 0.7) (layers F.Cu B.Cu) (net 5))
 (segment (start 133.75 130) (end 134.25 130) (width 0.25) (layer B.Cu) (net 5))
 (segment (start 132.75 129) (end 133.75 130) (width 0.25) (layer B.Cu) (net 5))
 (segment (start 132.75 128.721002) (end 132.75 129) (width 0.25) (layer B.Cu) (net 5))
 (segment (start 132.75 128.170972) (end 132.75 128.721002) (width 0.25) (layer B.Cu) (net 5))
 (segment (start 132.120286 128.096258) (end 132.675286 128.096258) (width 0.25) (layer B.Cu) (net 5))
 (segment (start 132.675286 128.096258) (end 132.75 128.170972) (width 0.25) (layer B.Cu) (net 5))
 (segment (start 133.25 127) (end 133.75 127.5) (width 0.25) (layer B.Cu) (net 12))
 (segment (start 133.75 127.5) (end 133.75 128.5) (width 0.25) (layer B.Cu) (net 12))
 (via (at 133.75 128.5) (size 1.2) (drill 0.7) (layers F.Cu B.Cu) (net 12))
 (segment (start 132.36903 127) (end 133.25 127) (width 0.25) (layer B.Cu) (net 12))
 (segment (start 126.25 127) (end 132.36903 127) (width 0.25) (layer B.Cu) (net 12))
 (segment (start 126.120286 127.129714) (end 126.25 127) (width 0.25) (layer B.Cu) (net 12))
 (segment (start 126.120286 128.096258) (end 126.120286 127.129714) (width 0.25) (layer B.Cu) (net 12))
 (segment (start 123.109028 126.5) (end 134.25 126.5) (width 0.25) (layer B.Cu) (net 15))
 (via (at 134.25 126.5) (size 1.2) (drill 0.7) (layers F.Cu B.Cu) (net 15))
 (segment (start 122.310286 124.816258) (end 122.310286 125.701258) (width 0.25) (layer B.Cu) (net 15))
 (segment (start 122.310286 125.701258) (end 123.109028 126.5) (width 0.25) (layer B.Cu) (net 15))
 (segment (start 133.75 125) (end 133.75 124.5) (width 0.25) (layer B.Cu) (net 3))
 (via (at 133.75 124.5) (size 1.2) (drill 0.7) (layers F.Cu B.Cu) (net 3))
 (segment (start 133.75 125.5) (end 133.75 125) (width 0.25) (layer B.Cu) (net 3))
 (segment (start 133.25 126) (end 133.75 125.5) (width 0.25) (layer B.Cu) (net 3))
 (segment (start 128.609028 126) (end 133.25 126) (width 0.25) (layer B.Cu) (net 3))
 (segment (start 128.310286 124.816258) (end 128.310286 125.701258) (width 0.25) (layer B.Cu) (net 3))
 (segment (start 128.310286 125.701258) (end 128.609028 126) (width 0.25) (layer B.Cu) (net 3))
 (segment (start 114.25 126.759738) (end 113.5 127.509738) (width 0.25) (layer B.Cu) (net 25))
 (segment (start 115.25 126.759738) (end 114.25 126.759738) (width 0.25) (layer B.Cu) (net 25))
 (segment (start 115.25 127.259738) (end 114.5 127.259738) (width 0.25) (layer B.Cu) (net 26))
 (segment (start 114.5 127.259738) (end 113.75 128.009738) (width 0.25) (layer B.Cu) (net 26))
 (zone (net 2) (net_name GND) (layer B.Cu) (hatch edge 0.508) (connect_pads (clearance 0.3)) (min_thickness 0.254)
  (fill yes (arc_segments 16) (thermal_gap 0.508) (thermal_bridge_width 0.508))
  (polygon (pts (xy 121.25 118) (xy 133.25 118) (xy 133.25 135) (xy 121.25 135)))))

